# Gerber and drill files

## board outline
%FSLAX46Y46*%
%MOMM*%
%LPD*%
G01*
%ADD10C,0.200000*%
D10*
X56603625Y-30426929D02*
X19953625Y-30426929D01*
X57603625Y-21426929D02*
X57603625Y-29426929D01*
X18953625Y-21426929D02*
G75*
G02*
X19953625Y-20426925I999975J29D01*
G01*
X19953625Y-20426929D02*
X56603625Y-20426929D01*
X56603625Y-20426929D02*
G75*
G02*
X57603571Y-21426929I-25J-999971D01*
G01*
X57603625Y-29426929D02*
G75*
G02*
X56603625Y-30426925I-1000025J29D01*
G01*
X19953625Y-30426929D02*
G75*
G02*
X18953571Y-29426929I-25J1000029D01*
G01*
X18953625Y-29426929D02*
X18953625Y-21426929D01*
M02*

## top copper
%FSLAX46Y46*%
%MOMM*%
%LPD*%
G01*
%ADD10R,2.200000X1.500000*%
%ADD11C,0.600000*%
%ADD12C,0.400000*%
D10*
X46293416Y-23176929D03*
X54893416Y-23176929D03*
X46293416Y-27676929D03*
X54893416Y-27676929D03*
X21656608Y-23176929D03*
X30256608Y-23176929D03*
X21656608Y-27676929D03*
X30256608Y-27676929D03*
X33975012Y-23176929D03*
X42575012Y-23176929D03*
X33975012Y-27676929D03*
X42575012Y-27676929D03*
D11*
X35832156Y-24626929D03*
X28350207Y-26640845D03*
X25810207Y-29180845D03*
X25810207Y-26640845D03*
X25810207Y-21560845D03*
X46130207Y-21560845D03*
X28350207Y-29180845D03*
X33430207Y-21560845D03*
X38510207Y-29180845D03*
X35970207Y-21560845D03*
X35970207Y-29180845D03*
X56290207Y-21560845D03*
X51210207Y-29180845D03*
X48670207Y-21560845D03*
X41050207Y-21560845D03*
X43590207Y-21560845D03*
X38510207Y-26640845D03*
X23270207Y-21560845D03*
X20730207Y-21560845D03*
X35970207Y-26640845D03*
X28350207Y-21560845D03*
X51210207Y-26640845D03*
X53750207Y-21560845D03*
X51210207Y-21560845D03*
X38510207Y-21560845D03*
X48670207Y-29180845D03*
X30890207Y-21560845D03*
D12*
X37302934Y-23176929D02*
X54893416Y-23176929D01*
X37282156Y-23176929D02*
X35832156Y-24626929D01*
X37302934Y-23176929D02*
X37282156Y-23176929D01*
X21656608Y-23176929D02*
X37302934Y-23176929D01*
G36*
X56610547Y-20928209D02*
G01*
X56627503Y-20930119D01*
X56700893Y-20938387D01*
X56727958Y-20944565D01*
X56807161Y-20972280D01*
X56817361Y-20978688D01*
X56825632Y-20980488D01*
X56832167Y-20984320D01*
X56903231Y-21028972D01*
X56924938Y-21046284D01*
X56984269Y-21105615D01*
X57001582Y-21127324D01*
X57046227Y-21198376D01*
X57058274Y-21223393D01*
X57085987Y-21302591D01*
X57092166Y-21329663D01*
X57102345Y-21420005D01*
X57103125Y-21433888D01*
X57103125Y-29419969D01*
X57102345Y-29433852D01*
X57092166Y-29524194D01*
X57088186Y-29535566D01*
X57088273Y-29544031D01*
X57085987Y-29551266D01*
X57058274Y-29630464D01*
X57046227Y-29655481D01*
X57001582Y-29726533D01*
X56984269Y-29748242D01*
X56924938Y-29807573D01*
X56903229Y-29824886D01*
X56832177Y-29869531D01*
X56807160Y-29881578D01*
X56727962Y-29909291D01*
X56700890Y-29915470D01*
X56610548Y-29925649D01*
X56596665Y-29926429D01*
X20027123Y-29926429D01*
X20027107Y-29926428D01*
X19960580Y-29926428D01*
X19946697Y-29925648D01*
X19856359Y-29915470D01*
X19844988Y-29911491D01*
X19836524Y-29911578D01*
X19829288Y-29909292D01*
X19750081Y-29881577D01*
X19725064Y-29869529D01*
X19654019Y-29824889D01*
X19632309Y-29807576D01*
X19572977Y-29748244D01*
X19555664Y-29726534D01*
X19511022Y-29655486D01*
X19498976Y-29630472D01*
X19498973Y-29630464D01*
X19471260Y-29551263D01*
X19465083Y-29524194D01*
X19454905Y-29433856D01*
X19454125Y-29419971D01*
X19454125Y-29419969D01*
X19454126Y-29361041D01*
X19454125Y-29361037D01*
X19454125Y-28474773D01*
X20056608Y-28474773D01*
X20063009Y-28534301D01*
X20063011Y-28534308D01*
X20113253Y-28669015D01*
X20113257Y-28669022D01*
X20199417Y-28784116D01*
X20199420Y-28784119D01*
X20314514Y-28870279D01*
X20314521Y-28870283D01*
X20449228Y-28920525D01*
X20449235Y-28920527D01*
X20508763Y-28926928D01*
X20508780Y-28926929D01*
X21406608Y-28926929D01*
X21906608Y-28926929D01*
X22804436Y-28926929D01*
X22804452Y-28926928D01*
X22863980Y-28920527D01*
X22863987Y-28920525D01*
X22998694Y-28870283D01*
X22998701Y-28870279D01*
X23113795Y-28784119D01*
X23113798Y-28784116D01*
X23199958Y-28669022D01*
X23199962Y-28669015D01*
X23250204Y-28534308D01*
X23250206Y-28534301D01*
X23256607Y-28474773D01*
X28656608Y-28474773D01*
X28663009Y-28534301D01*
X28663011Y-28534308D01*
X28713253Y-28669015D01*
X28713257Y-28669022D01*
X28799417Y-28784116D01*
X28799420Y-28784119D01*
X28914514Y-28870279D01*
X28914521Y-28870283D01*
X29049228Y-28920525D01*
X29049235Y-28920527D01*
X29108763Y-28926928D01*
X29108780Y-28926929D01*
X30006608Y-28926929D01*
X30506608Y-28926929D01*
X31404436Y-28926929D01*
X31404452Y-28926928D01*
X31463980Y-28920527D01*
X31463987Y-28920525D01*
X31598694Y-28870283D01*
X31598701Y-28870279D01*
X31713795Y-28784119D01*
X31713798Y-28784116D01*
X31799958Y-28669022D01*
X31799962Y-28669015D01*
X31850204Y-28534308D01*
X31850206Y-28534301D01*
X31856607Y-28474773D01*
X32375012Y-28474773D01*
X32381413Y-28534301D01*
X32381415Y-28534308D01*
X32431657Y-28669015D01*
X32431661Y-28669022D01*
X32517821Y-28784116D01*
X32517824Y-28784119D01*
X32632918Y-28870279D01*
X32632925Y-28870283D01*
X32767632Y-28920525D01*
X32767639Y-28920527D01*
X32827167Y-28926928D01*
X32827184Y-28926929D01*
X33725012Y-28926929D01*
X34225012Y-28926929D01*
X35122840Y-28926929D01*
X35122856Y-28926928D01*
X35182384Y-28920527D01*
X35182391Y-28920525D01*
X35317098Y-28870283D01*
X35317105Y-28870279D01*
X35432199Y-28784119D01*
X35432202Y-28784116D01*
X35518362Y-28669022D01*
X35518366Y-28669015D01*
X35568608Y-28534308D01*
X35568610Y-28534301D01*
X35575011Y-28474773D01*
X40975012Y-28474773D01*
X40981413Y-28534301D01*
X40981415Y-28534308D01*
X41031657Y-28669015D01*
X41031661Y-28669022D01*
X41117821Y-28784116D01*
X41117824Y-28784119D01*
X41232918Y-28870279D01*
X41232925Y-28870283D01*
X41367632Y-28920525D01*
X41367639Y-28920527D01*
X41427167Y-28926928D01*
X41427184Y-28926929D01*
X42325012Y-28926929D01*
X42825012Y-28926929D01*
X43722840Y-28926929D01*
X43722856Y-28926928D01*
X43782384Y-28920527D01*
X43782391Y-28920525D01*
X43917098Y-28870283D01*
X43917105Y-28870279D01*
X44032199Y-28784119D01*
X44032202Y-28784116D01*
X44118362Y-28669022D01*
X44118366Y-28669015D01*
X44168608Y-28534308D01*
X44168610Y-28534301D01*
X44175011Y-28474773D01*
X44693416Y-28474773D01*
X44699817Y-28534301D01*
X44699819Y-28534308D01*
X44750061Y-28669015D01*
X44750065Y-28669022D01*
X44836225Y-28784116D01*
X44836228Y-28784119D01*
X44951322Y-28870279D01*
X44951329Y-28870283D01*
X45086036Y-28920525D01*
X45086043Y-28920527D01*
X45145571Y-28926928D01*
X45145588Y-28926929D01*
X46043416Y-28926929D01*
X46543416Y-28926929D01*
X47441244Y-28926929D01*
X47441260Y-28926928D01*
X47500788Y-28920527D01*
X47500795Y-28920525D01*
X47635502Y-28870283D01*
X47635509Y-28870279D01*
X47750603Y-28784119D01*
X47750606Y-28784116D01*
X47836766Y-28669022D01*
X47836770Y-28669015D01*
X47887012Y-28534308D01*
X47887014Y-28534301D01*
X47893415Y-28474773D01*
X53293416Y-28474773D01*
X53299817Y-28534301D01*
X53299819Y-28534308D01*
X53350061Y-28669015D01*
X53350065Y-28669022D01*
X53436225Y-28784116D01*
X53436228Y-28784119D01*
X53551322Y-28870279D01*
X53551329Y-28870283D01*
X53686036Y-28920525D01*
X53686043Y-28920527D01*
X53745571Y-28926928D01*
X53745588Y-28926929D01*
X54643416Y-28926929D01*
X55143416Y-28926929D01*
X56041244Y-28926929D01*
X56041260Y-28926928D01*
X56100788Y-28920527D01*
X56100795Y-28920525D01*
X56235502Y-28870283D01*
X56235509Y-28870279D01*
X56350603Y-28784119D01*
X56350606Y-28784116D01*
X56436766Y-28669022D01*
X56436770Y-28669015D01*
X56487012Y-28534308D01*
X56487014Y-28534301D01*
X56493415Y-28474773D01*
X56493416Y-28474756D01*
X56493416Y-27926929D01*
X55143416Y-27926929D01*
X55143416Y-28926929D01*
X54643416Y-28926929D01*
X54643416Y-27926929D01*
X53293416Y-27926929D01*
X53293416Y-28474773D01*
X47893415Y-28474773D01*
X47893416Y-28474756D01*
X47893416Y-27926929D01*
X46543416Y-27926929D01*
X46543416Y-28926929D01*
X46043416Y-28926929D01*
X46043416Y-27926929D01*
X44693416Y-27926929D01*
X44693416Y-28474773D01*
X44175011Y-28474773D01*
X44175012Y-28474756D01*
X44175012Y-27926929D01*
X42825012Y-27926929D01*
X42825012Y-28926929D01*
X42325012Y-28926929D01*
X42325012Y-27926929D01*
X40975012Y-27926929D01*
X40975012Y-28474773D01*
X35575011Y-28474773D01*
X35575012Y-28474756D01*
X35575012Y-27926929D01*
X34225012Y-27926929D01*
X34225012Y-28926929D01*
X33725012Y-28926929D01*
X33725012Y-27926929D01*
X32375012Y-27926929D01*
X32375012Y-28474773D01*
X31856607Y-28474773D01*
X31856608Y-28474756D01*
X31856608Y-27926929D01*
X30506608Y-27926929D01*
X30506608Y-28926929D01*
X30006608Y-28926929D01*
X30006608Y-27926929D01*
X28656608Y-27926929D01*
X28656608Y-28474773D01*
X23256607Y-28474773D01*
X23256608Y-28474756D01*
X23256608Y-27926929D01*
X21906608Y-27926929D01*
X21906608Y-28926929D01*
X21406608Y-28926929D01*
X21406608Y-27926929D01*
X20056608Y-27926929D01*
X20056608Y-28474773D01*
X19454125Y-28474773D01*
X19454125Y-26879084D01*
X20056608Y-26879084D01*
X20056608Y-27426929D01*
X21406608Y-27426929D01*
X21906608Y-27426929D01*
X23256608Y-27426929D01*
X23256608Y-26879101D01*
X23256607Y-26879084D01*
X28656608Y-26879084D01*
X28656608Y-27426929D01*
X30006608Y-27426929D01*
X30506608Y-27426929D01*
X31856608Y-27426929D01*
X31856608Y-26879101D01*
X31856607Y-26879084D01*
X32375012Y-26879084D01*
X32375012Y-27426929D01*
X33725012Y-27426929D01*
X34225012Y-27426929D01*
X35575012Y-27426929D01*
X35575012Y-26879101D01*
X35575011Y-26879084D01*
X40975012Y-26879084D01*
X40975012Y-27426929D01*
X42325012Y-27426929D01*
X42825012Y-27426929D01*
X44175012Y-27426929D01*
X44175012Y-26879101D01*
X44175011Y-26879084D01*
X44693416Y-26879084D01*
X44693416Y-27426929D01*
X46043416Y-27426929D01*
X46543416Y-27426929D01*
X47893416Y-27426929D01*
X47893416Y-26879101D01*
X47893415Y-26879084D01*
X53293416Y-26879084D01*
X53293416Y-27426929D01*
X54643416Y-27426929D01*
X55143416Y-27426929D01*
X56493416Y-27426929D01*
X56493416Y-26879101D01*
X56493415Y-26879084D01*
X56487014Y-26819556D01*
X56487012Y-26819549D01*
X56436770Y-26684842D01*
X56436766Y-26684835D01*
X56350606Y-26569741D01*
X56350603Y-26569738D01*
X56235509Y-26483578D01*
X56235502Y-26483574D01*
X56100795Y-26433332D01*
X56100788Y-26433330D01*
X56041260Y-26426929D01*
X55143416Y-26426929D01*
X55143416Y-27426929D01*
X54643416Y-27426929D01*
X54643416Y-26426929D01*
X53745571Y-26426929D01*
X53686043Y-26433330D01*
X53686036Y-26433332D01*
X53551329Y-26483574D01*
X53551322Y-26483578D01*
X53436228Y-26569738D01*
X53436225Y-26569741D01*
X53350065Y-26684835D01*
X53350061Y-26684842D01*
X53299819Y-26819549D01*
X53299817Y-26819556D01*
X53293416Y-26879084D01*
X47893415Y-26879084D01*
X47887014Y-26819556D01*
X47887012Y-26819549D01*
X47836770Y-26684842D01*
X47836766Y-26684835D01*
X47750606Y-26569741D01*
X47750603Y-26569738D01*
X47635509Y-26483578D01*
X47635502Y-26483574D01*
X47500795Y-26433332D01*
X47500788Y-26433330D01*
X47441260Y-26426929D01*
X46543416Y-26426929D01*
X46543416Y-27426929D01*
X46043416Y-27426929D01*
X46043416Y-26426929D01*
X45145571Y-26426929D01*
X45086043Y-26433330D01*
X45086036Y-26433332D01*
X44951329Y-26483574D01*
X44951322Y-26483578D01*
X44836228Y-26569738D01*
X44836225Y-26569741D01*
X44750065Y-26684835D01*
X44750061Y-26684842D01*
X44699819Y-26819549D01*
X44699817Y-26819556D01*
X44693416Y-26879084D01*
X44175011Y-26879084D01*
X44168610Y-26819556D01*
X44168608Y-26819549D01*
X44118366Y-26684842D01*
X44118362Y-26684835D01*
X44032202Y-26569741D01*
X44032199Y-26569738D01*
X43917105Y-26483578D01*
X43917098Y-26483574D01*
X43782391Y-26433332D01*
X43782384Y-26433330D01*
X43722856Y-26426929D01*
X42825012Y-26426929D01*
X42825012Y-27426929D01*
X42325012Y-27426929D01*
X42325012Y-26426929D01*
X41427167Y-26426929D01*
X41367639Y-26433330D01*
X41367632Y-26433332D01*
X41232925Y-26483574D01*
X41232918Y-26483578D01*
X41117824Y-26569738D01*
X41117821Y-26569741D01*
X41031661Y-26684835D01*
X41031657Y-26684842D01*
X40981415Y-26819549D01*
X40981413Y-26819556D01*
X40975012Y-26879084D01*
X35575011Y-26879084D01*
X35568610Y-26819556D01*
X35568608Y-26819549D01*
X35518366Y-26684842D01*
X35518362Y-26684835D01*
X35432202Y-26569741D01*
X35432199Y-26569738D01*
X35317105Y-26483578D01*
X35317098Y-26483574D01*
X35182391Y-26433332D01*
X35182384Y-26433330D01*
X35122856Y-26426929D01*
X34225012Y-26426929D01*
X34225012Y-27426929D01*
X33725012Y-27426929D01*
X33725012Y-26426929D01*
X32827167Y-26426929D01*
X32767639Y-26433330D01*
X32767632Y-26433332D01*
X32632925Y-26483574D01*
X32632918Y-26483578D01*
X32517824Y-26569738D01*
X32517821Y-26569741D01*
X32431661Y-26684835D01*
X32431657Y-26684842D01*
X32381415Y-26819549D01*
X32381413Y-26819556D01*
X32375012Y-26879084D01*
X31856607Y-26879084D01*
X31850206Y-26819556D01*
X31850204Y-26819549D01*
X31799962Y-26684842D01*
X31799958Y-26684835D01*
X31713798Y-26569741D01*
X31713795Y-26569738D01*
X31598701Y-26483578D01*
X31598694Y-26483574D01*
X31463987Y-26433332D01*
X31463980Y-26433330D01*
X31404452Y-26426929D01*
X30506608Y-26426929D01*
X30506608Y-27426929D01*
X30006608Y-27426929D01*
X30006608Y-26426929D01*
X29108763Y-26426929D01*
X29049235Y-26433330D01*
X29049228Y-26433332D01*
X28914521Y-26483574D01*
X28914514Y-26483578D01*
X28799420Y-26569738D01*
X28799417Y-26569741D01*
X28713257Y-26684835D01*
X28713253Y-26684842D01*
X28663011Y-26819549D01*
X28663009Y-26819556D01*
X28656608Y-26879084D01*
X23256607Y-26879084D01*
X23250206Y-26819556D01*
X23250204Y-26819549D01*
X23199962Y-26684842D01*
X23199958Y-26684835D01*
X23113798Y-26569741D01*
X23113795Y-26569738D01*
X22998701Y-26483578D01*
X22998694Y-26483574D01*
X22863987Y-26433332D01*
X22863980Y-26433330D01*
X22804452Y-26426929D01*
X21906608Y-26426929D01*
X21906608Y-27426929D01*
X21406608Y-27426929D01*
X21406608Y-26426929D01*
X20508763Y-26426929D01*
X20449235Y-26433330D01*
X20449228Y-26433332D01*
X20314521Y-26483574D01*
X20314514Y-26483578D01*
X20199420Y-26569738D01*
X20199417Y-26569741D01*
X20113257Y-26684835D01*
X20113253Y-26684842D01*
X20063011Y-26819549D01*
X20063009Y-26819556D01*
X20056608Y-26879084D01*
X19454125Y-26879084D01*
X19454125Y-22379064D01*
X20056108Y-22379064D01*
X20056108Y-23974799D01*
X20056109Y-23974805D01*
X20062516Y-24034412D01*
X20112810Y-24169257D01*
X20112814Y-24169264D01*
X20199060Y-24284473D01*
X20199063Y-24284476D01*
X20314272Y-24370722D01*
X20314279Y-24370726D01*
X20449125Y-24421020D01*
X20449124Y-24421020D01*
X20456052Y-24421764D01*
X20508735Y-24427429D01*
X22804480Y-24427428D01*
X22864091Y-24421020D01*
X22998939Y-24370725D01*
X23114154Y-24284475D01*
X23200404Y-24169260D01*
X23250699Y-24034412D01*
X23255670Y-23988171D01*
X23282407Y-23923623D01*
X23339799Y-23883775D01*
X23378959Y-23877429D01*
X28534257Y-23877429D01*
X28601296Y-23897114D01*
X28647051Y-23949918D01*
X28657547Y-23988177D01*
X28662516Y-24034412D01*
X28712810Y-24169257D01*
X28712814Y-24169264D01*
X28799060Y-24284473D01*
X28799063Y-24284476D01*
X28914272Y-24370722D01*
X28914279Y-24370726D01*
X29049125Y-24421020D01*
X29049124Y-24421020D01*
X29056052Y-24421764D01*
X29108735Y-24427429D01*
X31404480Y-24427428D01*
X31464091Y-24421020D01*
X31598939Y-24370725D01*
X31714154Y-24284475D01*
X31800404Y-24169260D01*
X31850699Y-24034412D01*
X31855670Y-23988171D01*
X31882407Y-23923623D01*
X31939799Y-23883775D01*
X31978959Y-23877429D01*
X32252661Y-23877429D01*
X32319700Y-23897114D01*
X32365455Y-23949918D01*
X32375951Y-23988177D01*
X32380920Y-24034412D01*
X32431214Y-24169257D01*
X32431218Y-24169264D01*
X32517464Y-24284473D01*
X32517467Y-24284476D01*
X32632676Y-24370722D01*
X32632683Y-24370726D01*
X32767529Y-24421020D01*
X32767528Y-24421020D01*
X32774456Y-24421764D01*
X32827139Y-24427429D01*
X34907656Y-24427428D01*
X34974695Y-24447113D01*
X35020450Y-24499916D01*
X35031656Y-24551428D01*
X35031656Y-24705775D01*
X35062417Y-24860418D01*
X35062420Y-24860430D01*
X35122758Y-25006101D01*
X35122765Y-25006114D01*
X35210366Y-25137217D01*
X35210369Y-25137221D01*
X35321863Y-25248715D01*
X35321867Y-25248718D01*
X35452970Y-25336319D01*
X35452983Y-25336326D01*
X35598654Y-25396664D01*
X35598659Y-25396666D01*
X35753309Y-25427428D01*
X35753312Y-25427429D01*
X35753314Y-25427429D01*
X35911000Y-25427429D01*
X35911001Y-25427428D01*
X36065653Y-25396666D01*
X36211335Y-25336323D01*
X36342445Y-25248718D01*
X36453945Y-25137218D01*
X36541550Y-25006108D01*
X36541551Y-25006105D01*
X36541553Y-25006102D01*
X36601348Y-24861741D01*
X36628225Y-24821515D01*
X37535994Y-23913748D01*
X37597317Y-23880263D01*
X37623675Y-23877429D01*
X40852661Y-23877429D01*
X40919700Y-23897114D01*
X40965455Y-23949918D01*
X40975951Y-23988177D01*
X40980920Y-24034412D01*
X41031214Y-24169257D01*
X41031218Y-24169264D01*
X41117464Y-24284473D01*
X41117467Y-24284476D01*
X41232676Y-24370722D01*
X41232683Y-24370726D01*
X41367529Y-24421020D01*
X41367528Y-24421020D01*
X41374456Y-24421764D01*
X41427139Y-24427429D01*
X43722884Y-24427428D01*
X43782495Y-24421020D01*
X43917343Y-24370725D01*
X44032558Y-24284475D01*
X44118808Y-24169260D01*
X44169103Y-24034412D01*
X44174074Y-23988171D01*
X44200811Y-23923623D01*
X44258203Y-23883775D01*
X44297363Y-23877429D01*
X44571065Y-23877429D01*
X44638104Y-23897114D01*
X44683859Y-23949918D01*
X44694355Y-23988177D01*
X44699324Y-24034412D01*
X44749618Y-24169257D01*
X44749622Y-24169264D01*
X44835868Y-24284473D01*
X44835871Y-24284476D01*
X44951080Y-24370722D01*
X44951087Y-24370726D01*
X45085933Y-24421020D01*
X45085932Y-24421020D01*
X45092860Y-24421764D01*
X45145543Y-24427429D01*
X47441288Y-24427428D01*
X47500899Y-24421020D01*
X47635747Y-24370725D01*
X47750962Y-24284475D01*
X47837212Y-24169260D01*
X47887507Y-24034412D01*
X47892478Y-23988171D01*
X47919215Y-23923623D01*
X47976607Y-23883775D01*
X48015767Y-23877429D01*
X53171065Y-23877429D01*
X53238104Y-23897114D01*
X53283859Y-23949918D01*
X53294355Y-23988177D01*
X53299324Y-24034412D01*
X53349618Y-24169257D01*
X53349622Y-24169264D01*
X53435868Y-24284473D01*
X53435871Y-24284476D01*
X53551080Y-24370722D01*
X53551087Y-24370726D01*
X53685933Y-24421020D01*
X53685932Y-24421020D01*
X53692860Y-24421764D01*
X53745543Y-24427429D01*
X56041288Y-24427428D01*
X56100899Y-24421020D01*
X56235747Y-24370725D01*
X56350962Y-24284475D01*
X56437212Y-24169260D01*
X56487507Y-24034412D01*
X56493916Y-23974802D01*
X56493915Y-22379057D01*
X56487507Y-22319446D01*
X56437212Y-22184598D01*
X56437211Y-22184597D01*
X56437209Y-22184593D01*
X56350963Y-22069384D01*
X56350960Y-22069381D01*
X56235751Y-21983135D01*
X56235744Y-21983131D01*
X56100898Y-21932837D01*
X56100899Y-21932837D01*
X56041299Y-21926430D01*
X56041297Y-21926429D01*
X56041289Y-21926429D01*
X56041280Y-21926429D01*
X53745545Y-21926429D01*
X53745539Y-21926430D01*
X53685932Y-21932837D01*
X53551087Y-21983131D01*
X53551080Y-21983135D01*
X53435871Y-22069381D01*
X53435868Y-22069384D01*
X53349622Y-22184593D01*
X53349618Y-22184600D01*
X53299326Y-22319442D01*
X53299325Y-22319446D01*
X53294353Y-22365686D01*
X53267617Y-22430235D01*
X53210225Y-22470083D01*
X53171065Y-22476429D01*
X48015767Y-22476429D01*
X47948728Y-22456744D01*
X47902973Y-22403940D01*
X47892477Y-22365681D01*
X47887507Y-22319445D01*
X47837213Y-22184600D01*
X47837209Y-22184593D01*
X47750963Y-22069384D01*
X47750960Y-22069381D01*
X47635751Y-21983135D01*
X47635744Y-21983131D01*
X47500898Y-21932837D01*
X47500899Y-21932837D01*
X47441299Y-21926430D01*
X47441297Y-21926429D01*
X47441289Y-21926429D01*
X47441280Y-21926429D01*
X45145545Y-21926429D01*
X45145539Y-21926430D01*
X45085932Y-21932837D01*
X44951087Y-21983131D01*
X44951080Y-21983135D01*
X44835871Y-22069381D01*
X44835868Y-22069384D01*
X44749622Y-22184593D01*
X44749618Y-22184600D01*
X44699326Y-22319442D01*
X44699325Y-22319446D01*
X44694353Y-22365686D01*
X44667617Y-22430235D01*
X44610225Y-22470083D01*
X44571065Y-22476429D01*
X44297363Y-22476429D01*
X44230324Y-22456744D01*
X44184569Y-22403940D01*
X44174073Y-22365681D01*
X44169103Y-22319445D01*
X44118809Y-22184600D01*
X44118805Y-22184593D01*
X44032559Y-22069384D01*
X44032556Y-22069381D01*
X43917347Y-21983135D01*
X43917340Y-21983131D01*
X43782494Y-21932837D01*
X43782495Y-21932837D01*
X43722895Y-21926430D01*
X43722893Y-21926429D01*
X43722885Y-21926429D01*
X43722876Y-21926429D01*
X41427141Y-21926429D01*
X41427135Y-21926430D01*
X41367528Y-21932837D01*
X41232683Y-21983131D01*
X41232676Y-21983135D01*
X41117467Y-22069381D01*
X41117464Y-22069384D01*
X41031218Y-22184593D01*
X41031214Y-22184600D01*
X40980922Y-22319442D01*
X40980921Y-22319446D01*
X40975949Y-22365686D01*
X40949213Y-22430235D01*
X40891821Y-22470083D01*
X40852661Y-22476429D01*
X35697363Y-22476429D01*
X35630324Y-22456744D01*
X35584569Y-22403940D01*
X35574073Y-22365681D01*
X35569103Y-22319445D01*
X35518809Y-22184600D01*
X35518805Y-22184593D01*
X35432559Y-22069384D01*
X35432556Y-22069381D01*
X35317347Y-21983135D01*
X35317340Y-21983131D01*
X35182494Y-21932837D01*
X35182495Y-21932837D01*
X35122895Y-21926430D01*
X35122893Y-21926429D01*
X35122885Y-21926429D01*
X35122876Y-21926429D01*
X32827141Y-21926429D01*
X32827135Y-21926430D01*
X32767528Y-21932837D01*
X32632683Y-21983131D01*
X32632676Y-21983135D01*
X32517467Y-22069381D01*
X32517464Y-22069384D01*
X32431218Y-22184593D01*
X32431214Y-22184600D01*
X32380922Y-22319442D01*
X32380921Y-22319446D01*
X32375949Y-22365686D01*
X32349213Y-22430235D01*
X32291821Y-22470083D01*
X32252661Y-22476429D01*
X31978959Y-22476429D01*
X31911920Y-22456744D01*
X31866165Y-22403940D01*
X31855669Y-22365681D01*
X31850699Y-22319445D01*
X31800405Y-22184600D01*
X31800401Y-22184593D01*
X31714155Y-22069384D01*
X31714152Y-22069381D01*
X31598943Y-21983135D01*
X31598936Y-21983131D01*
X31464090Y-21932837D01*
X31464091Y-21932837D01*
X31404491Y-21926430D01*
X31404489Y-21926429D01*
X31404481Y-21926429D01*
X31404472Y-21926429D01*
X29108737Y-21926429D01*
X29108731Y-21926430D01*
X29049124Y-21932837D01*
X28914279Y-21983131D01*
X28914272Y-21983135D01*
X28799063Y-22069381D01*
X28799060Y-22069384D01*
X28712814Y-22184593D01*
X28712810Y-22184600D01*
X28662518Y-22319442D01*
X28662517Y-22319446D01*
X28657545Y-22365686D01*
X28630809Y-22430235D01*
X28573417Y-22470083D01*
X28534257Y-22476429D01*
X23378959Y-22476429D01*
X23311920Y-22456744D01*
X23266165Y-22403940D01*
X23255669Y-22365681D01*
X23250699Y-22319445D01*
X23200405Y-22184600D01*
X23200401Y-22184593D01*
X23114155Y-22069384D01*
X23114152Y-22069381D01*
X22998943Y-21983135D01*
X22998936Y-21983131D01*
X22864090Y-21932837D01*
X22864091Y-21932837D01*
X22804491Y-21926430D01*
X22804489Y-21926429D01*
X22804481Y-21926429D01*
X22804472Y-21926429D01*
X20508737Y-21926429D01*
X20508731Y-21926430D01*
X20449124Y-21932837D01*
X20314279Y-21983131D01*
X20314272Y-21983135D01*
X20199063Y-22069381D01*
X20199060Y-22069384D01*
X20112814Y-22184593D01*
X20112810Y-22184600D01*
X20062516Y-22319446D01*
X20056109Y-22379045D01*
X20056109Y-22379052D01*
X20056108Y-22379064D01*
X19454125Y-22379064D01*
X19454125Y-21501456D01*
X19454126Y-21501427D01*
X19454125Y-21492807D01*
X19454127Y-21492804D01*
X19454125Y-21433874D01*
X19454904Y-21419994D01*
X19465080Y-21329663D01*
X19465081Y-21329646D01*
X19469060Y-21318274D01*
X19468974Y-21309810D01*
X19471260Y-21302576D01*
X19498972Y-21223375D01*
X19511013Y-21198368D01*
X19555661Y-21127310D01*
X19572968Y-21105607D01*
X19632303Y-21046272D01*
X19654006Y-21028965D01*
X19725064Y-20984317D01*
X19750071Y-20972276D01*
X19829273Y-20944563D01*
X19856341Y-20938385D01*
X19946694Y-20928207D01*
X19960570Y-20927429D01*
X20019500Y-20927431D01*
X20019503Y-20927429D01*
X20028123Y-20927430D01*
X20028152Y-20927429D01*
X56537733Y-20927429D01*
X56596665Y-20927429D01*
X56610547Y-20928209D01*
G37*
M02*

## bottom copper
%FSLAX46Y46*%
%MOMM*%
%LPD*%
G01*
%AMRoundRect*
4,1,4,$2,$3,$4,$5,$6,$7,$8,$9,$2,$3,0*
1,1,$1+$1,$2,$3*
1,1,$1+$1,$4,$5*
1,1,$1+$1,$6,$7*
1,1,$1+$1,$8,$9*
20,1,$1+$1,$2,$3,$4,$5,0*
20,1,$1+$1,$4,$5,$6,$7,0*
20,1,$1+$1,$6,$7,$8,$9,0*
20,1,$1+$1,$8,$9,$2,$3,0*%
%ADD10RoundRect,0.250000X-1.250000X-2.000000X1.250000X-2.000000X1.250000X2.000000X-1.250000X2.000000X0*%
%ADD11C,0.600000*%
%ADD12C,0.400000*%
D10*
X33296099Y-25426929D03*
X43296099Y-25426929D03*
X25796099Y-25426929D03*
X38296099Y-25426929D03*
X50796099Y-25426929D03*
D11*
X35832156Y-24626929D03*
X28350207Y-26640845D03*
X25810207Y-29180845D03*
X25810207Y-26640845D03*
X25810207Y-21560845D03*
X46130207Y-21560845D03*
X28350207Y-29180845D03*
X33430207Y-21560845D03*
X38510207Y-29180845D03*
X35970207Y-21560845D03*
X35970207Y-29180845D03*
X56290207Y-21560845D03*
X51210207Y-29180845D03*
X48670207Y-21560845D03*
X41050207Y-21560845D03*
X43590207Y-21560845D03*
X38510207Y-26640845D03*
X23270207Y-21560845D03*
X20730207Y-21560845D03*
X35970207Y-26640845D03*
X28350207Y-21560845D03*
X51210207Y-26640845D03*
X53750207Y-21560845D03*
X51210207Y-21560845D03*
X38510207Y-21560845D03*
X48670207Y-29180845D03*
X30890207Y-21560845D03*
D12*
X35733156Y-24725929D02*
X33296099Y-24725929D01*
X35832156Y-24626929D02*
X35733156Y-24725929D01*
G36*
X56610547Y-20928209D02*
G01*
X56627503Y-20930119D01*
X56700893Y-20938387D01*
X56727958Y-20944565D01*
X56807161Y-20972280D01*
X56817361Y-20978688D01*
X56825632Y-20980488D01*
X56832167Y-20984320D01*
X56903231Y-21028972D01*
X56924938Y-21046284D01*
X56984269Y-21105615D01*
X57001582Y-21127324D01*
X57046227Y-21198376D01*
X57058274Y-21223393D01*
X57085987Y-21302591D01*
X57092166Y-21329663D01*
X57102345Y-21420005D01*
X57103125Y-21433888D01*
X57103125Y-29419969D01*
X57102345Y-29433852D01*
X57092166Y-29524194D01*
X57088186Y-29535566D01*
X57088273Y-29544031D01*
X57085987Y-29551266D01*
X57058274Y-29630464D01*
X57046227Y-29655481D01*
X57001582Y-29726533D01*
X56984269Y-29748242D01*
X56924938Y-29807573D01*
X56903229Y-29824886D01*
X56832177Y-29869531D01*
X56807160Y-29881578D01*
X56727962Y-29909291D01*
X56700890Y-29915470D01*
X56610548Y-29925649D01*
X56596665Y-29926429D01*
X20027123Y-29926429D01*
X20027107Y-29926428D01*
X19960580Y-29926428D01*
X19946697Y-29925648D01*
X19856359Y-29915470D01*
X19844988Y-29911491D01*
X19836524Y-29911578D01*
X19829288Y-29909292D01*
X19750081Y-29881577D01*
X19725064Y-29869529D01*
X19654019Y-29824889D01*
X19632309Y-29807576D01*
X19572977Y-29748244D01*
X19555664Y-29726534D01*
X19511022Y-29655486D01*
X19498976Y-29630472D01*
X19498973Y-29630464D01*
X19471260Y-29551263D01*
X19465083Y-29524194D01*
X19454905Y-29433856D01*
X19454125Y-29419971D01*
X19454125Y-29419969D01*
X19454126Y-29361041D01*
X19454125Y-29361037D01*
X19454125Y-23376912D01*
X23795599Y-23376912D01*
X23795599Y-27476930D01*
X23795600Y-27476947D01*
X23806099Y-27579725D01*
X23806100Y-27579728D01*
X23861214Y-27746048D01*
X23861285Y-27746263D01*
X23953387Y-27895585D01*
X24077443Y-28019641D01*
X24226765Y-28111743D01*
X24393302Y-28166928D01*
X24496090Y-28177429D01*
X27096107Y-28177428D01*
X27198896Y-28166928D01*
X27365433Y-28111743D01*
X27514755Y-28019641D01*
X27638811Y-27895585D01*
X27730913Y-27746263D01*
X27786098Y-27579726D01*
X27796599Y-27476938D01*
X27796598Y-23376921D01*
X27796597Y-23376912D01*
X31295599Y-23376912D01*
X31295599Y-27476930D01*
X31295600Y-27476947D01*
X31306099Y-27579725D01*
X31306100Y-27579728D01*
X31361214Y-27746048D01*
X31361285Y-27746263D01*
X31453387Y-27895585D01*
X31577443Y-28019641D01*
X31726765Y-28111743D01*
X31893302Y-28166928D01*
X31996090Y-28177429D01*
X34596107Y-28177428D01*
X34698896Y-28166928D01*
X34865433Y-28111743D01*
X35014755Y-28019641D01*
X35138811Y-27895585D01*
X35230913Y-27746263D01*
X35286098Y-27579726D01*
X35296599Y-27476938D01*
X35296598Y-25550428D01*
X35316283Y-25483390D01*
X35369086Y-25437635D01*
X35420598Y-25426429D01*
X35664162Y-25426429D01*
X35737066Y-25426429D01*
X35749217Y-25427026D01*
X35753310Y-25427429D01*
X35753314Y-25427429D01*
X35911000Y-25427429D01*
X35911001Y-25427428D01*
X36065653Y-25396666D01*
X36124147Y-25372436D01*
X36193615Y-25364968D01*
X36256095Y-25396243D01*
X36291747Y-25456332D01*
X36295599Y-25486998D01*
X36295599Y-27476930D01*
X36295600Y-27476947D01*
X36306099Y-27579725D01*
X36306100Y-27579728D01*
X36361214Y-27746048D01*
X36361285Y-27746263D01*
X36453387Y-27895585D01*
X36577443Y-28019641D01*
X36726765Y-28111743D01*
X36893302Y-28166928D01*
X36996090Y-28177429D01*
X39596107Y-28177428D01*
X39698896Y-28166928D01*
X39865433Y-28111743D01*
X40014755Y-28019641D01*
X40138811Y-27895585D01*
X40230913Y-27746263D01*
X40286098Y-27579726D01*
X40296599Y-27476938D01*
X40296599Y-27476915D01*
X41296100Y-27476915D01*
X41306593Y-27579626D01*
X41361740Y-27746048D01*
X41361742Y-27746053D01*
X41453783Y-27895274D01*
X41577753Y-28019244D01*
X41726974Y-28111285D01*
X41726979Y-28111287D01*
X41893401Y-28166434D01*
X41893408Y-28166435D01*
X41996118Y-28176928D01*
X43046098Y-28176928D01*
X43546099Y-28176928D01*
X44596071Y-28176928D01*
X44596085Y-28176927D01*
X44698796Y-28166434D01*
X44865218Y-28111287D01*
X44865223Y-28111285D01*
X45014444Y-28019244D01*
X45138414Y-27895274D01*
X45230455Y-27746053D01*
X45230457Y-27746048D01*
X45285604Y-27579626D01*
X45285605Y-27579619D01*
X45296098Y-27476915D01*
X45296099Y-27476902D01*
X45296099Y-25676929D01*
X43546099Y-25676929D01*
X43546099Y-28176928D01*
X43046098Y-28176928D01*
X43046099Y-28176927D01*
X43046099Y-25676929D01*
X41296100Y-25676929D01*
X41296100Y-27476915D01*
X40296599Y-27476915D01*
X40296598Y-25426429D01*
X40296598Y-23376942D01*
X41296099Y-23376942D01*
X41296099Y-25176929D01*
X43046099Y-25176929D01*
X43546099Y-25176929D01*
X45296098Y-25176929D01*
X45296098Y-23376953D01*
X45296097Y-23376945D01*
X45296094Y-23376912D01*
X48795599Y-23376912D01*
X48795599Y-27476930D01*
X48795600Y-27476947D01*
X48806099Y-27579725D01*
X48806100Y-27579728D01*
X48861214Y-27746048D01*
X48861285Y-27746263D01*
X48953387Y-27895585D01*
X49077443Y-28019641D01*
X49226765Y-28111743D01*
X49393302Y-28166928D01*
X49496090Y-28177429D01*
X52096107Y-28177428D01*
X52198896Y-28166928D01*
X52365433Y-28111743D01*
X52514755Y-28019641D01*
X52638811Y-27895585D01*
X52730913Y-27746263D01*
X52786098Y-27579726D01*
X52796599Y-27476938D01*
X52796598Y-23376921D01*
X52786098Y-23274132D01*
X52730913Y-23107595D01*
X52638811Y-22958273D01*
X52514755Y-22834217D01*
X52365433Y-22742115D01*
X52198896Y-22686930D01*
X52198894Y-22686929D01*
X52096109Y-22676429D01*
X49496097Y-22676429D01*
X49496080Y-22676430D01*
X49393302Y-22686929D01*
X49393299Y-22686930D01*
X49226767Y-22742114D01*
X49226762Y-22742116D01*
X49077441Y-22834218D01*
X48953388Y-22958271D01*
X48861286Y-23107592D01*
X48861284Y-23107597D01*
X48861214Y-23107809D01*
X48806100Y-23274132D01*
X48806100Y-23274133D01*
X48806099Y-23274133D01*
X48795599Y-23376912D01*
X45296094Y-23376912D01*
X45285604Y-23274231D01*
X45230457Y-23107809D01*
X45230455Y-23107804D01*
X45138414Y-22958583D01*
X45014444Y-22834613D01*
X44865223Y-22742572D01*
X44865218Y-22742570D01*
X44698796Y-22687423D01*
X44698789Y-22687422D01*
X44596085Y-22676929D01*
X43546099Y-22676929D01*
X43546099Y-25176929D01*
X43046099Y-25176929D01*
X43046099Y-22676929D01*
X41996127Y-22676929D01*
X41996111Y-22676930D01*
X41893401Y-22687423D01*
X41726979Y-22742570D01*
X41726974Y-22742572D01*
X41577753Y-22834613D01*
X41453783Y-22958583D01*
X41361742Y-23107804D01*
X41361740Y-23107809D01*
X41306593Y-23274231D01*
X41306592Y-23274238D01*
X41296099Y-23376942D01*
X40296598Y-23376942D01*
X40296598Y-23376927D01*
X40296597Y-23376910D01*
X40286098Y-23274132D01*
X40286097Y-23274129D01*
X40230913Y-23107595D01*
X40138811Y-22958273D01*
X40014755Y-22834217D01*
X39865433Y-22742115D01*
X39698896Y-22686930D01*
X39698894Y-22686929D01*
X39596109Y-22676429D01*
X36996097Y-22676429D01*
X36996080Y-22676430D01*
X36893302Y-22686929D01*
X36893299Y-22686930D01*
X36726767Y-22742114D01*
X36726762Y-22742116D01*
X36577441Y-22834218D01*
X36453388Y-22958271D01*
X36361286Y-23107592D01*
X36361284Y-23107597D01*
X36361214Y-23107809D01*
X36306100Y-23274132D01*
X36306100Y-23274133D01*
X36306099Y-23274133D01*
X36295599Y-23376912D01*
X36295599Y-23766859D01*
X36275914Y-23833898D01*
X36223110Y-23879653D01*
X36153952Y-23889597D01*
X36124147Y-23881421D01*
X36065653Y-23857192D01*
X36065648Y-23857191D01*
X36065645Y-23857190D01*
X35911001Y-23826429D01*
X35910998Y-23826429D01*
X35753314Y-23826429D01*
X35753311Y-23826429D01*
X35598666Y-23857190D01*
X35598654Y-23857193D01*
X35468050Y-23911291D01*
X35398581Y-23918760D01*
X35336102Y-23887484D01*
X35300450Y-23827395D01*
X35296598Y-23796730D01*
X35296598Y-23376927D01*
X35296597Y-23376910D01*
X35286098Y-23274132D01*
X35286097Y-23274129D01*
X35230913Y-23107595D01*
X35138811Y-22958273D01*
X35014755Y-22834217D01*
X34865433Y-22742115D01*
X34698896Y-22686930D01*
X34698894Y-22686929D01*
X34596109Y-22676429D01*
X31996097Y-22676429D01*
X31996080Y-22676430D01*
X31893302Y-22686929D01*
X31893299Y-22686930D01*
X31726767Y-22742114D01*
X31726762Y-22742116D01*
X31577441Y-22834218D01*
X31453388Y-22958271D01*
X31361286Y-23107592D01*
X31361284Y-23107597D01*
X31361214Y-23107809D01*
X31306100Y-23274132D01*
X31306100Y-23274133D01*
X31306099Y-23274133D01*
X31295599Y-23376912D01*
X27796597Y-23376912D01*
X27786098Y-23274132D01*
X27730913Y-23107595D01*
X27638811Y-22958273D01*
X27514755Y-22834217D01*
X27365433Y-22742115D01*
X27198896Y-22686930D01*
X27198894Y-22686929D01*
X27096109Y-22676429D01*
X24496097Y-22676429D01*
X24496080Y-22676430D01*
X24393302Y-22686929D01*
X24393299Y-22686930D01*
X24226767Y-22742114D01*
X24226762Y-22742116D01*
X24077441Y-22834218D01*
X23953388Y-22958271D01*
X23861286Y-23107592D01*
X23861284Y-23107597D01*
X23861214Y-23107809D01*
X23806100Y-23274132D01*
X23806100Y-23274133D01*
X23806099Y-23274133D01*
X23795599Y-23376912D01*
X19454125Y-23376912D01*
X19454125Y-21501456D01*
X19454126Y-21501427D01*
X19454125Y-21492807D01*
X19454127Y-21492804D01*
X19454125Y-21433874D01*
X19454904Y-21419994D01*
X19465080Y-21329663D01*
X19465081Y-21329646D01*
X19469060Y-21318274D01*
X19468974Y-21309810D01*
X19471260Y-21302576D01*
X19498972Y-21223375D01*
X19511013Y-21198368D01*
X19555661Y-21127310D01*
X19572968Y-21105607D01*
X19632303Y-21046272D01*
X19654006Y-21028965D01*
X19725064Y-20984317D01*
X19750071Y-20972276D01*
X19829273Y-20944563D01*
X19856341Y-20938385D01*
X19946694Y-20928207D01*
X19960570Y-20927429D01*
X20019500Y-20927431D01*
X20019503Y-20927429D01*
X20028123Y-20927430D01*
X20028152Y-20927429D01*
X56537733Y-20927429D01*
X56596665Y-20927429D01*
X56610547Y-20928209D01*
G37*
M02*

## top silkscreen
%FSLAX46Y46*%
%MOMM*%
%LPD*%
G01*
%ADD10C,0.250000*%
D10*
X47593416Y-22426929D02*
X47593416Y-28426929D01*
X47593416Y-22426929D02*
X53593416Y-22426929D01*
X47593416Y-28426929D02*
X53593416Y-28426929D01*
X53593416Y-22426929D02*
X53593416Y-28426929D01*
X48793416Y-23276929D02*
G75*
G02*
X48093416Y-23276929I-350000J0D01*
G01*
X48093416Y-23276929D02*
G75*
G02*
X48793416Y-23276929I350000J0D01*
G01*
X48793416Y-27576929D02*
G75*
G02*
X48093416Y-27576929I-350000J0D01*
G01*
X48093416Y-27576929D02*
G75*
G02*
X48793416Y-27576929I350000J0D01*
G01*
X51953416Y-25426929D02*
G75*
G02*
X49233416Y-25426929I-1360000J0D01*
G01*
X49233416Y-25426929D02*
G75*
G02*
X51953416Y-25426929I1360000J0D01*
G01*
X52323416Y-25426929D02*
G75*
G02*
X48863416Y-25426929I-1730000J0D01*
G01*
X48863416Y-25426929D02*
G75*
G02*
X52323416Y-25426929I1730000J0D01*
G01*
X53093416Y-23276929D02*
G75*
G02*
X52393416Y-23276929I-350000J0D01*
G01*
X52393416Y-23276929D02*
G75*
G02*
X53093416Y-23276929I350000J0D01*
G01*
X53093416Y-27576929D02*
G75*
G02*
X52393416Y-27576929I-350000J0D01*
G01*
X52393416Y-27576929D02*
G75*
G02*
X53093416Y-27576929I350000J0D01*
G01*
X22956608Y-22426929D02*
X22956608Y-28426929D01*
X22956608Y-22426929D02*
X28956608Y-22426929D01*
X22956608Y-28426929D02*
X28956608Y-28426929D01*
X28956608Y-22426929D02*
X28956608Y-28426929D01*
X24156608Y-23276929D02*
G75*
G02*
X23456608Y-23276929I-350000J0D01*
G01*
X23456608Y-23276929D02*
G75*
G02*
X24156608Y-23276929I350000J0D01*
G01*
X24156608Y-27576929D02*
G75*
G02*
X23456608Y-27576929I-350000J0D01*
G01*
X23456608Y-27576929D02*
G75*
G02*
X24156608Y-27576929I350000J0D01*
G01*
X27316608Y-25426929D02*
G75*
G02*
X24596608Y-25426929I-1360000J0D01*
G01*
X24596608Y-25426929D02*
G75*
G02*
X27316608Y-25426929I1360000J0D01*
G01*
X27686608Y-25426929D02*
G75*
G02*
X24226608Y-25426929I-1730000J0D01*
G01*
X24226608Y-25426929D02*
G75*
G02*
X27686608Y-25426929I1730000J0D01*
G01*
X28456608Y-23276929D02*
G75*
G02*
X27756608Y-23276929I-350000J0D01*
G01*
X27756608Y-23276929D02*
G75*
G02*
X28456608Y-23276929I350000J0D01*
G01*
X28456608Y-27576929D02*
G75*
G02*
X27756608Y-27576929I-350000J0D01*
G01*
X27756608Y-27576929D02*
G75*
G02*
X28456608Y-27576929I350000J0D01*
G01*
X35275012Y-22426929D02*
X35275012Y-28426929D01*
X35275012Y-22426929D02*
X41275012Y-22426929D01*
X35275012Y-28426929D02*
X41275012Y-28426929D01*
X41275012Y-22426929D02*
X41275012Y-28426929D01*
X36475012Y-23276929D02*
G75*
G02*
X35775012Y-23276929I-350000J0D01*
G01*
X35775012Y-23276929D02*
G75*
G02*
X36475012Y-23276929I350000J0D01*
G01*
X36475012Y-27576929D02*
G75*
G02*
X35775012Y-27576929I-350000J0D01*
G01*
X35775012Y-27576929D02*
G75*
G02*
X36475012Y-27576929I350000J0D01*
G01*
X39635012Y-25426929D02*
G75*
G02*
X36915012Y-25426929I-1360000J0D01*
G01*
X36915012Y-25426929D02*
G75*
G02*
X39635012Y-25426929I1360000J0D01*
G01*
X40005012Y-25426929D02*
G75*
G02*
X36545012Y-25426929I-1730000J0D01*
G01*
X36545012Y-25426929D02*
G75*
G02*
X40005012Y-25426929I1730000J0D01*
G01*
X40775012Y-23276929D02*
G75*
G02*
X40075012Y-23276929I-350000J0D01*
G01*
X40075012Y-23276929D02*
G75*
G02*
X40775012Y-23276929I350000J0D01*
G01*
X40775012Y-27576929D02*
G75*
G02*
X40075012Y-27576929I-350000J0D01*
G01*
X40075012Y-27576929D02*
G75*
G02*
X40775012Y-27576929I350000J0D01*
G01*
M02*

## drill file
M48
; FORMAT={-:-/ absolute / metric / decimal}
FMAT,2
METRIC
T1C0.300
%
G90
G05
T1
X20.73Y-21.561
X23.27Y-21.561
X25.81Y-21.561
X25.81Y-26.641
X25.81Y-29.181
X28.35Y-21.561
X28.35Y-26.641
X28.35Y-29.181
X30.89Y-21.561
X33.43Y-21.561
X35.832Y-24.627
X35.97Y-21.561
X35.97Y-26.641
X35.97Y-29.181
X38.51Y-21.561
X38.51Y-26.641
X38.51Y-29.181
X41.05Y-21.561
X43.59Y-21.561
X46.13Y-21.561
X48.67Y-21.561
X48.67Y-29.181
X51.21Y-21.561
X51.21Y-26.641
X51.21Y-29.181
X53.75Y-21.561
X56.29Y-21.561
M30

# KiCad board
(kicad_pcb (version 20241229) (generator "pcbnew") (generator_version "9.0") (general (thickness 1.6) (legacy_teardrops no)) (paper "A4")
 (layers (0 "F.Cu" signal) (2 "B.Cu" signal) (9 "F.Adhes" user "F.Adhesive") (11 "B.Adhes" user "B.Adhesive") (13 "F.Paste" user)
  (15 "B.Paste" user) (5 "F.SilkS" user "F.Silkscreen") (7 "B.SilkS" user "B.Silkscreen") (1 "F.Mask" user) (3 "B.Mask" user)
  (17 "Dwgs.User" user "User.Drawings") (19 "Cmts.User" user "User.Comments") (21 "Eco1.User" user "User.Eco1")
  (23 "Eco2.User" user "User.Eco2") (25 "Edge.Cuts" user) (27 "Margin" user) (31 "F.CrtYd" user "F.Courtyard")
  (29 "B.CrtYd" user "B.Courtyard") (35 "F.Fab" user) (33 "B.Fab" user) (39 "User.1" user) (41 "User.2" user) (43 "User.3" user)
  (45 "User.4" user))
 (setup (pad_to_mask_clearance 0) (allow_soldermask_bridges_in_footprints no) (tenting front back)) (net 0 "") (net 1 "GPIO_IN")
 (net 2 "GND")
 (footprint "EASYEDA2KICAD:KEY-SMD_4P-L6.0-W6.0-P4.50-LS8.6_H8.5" (layer "F.Cu") (at 50.593416 25.426929)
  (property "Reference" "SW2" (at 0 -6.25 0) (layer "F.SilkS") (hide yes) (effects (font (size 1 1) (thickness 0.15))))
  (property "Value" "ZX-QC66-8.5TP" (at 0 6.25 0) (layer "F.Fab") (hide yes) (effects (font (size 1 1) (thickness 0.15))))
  (fp_line (start -3 -3) (end -3 3) (stroke (width 0.25) (type solid)) (layer "F.SilkS"))
  (fp_line (start -3 -3) (end 3 -3) (stroke (width 0.25) (type solid)) (layer "F.SilkS"))
  (fp_line (start -3 3) (end 3 3) (stroke (width 0.25) (type solid)) (layer "F.SilkS"))
  (fp_line (start 3 -3) (end 3 3) (stroke (width 0.25) (type solid)) (layer "F.SilkS"))
  (fp_circle (center -2.15 -2.15) (end -1.8 -2.15) (stroke (width 0.25) (type solid)) (fill no) (layer "F.SilkS"))
  (fp_circle (center -2.15 2.15) (end -1.8 2.15) (stroke (width 0.25) (type solid)) (fill no) (layer "F.SilkS"))
  (fp_circle (center 0 0) (end 1.36 0) (stroke (width 0.25) (type solid)) (fill no) (layer "F.SilkS"))
  (fp_circle (center 0 0) (end 1.73 0) (stroke (width 0.25) (type solid)) (fill no) (layer "F.SilkS"))
  (fp_circle (center 2.15 -2.15) (end 2.5 -2.15) (stroke (width 0.25) (type solid)) (fill no) (layer "F.SilkS"))
  (fp_circle (center 2.15 2.15) (end 2.5 2.15) (stroke (width 0.25) (type solid)) (fill no) (layer "F.SilkS"))
  (pad "1" smd rect (at -4.3 -2.25) (size 2.2 1.5) (layers "F.Cu" "F.Mask" "F.Paste") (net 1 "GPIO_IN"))
  (pad "2" smd rect (at 4.3 -2.25) (size 2.2 1.5) (layers "F.Cu" "F.Mask" "F.Paste") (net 1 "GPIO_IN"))
  (pad "3" smd rect (at -4.3 2.25) (size 2.2 1.5) (layers "F.Cu" "F.Mask" "F.Paste") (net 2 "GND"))
  (pad "4" smd rect (at 4.3 2.25) (size 2.2 1.5) (layers "F.Cu" "F.Mask" "F.Paste") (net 2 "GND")))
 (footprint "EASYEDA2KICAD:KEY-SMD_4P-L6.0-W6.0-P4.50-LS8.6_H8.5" (layer "F.Cu") (at 25.956608 25.426929)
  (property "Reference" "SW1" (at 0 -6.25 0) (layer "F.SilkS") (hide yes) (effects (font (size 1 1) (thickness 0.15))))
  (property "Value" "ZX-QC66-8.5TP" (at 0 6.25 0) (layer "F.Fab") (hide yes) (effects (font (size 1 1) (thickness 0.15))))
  (fp_line (start -3 -3) (end -3 3) (stroke (width 0.25) (type solid)) (layer "F.SilkS"))
  (fp_line (start -3 -3) (end 3 -3) (stroke (width 0.25) (type solid)) (layer "F.SilkS"))
  (fp_line (start -3 3) (end 3 3) (stroke (width 0.25) (type solid)) (layer "F.SilkS"))
  (fp_line (start 3 -3) (end 3 3) (stroke (width 0.25) (type solid)) (layer "F.SilkS"))
  (fp_circle (center -2.15 -2.15) (end -1.8 -2.15) (stroke (width 0.25) (type solid)) (fill no) (layer "F.SilkS"))
  (fp_circle (center -2.15 2.15) (end -1.8 2.15) (stroke (width 0.25) (type solid)) (fill no) (layer "F.SilkS"))
  (fp_circle (center 0 0) (end 1.36 0) (stroke (width 0.25) (type solid)) (fill no) (layer "F.SilkS"))
  (fp_circle (center 0 0) (end 1.73 0) (stroke (width 0.25) (type solid)) (fill no) (layer "F.SilkS"))
  (fp_circle (center 2.15 -2.15) (end 2.5 -2.15) (stroke (width 0.25) (type solid)) (fill no) (layer "F.SilkS"))
  (fp_circle (center 2.15 2.15) (end 2.5 2.15) (stroke (width 0.25) (type solid)) (fill no) (layer "F.SilkS"))
  (pad "1" smd rect (at -4.3 -2.25) (size 2.2 1.5) (layers "F.Cu" "F.Mask" "F.Paste") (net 1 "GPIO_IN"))
  (pad "2" smd rect (at 4.3 -2.25) (size 2.2 1.5) (layers "F.Cu" "F.Mask" "F.Paste") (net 1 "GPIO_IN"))
  (pad "3" smd rect (at -4.3 2.25) (size 2.2 1.5) (layers "F.Cu" "F.Mask" "F.Paste") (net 2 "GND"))
  (pad "4" smd rect (at 4.3 2.25) (size 2.2 1.5) (layers "F.Cu" "F.Mask" "F.Paste") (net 2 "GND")))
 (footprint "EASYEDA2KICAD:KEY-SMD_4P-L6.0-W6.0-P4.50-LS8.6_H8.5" (layer "F.Cu") (at 38.275012 25.426929)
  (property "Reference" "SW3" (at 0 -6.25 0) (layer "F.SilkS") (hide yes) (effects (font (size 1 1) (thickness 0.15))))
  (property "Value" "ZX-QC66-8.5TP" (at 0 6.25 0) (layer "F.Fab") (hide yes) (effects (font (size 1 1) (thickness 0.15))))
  (fp_line (start -3 -3) (end -3 3) (stroke (width 0.25) (type solid)) (layer "F.SilkS"))
  (fp_line (start -3 -3) (end 3 -3) (stroke (width 0.25) (type solid)) (layer "F.SilkS"))
  (fp_line (start -3 3) (end 3 3) (stroke (width 0.25) (type solid)) (layer "F.SilkS"))
  (fp_line (start 3 -3) (end 3 3) (stroke (width 0.25) (type solid)) (layer "F.SilkS"))
  (fp_circle (center -2.15 -2.15) (end -1.8 -2.15) (stroke (width 0.25) (type solid)) (fill no) (layer "F.SilkS"))
  (fp_circle (center -2.15 2.15) (end -1.8 2.15) (stroke (width 0.25) (type solid)) (fill no) (layer "F.SilkS"))
  (fp_circle (center 0 0) (end 1.36 0) (stroke (width 0.25) (type solid)) (fill no) (layer "F.SilkS"))
  (fp_circle (center 0 0) (end 1.73 0) (stroke (width 0.25) (type solid)) (fill no) (layer "F.SilkS"))
  (fp_circle (center 2.15 -2.15) (end 2.5 -2.15) (stroke (width 0.25) (type solid)) (fill no) (layer "F.SilkS"))
  (fp_circle (center 2.15 2.15) (end 2.5 2.15) (stroke (width 0.25) (type solid)) (fill no) (layer "F.SilkS"))
  (pad "1" smd rect (at -4.3 -2.25) (size 2.2 1.5) (layers "F.Cu" "F.Mask" "F.Paste") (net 1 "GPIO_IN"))
  (pad "2" smd rect (at 4.3 -2.25) (size 2.2 1.5) (layers "F.Cu" "F.Mask" "F.Paste") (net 1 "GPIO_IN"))
  (pad "3" smd rect (at -4.3 2.25) (size 2.2 1.5) (layers "F.Cu" "F.Mask" "F.Paste") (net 2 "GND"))
  (pad "4" smd rect (at 4.3 2.25) (size 2.2 1.5) (layers "F.Cu" "F.Mask" "F.Paste") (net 2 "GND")))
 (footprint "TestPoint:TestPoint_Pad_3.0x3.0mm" (layer "B.Cu") (at 38.296099 25.426929)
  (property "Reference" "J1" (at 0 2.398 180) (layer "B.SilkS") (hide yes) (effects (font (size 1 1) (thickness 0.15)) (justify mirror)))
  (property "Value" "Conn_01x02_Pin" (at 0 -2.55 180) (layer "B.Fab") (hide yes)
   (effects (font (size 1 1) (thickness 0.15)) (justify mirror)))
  (pad "1" smd roundrect (at -5 0) (size 3 4.5) (layers "B.Cu" "B.Mask") (roundrect_rratio 0.08333333333) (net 1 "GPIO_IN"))
  (pad "2" smd roundrect (at 5 0) (size 3 4.5) (layers "B.Cu" "B.Mask") (roundrect_rratio 0.08333333333) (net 2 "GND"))
  (pad "3" smd roundrect (at -12.5 0) (size 3 4.5) (layers "B.Cu" "B.Mask") (roundrect_rratio 0.08333333333))
  (pad "3" smd roundrect (at 0 0) (size 3 4.5) (layers "B.Cu" "B.Mask") (roundrect_rratio 0.08333333333))
  (pad "3" smd roundrect (at 12.5 0) (size 3 4.5) (layers "B.Cu" "B.Mask") (roundrect_rratio 0.08333333333)))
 (gr_line (start 56.603625 30.426929) (end 19.953625 30.426929) (stroke (width 0.2) (type default)) (layer "Edge.Cuts"))
 (gr_line (start 57.603625 21.426929) (end 57.603625 29.426929) (stroke (width 0.2) (type default)) (layer "Edge.Cuts"))
 (gr_arc (start 18.953625 21.426929) (mid 19.246509 20.719812) (end 19.953625 20.426929) (stroke (width 0.2) (type default))
  (layer "Edge.Cuts"))
 (gr_line (start 19.953625 20.426929) (end 56.603625 20.426929) (stroke (width 0.2) (type default)) (layer "Edge.Cuts"))
 (gr_arc (start 56.603625 20.426929) (mid 57.310732 20.719822) (end 57.603625 21.426929) (stroke (width 0.2) (type default))
  (layer "Edge.Cuts"))
 (gr_arc (start 57.603625 29.426929) (mid 57.310732 30.134036) (end 56.603625 30.426929) (stroke (width 0.2) (type default))
  (layer "Edge.Cuts"))
 (gr_arc (start 19.953625 30.426929) (mid 19.246515 30.134037) (end 18.953625 29.426929) (stroke (width 0.2) (type default))
  (layer "Edge.Cuts"))
 (gr_line (start 18.953625 29.426929) (end 18.953625 21.426929) (stroke (width 0.2) (type default)) (layer "Edge.Cuts"))
 (segment (start 37.302934 23.176929) (end 54.893416 23.176929) (width 0.4) (layer "F.Cu") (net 1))
 (segment (start 37.282156 23.176929) (end 35.832156 24.626929) (width 0.4) (layer "F.Cu") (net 1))
 (segment (start 37.302934 23.176929) (end 37.282156 23.176929) (width 0.4) (layer "F.Cu") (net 1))
 (segment (start 21.656608 23.176929) (end 37.302934 23.176929) (width 0.4) (layer "F.Cu") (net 1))
 (via (at 35.832156 24.626929) (size 0.6) (drill 0.3) (layers "F.Cu" "B.Cu") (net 1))
 (segment (start 35.733156 24.725929) (end 33.296099 24.725929) (width 0.4) (layer "B.Cu") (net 1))
 (segment (start 35.832156 24.626929) (end 35.733156 24.725929) (width 0.4) (layer "B.Cu") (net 1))
 (via (at 28.350207 26.640845) (size 0.6) (drill 0.3) (layers "F.Cu" "B.Cu") (free yes) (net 2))
 (via (at 25.810207 29.180845) (size 0.6) (drill 0.3) (layers "F.Cu" "B.Cu") (free yes) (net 2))
 (via (at 25.810207 26.640845) (size 0.6) (drill 0.3) (layers "F.Cu" "B.Cu") (free yes) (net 2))
 (via (at 25.810207 21.560845) (size 0.6) (drill 0.3) (layers "F.Cu" "B.Cu") (free yes) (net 2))
 (via (at 46.130207 21.560845) (size 0.6) (drill 0.3) (layers "F.Cu" "B.Cu") (free yes) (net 2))
 (via (at 28.350207 29.180845) (size 0.6) (drill 0.3) (layers "F.Cu" "B.Cu") (free yes) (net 2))
 (via (at 33.430207 21.560845) (size 0.6) (drill 0.3) (layers "F.Cu" "B.Cu") (free yes) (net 2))
 (via (at 38.510207 29.180845) (size 0.6) (drill 0.3) (layers "F.Cu" "B.Cu") (free yes) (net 2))
 (via (at 35.970207 21.560845) (size 0.6) (drill 0.3) (layers "F.Cu" "B.Cu") (free yes) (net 2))
 (via (at 35.970207 29.180845) (size 0.6) (drill 0.3) (layers "F.Cu" "B.Cu") (free yes) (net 2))
 (via (at 56.290207 21.560845) (size 0.6) (drill 0.3) (layers "F.Cu" "B.Cu") (free yes) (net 2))
 (via (at 51.210207 29.180845) (size 0.6) (drill 0.3) (layers "F.Cu" "B.Cu") (free yes) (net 2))
 (via (at 48.670207 21.560845) (size 0.6) (drill 0.3) (layers "F.Cu" "B.Cu") (free yes) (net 2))
 (via (at 41.050207 21.560845) (size 0.6) (drill 0.3) (layers "F.Cu" "B.Cu") (free yes) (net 2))
 (via (at 43.590207 21.560845) (size 0.6) (drill 0.3) (layers "F.Cu" "B.Cu") (free yes) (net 2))
 (via (at 38.510207 26.640845) (size 0.6) (drill 0.3) (layers "F.Cu" "B.Cu") (free yes) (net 2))
 (via (at 23.270207 21.560845) (size 0.6) (drill 0.3) (layers "F.Cu" "B.Cu") (free yes) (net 2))
 (via (at 20.730207 21.560845) (size 0.6) (drill 0.3) (layers "F.Cu" "B.Cu") (free yes) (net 2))
 (via (at 35.970207 26.640845) (size 0.6) (drill 0.3) (layers "F.Cu" "B.Cu") (free yes) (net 2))
 (via (at 28.350207 21.560845) (size 0.6) (drill 0.3) (layers "F.Cu" "B.Cu") (free yes) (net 2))
 (via (at 51.210207 26.640845) (size 0.6) (drill 0.3) (layers "F.Cu" "B.Cu") (free yes) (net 2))
 (via (at 53.750207 21.560845) (size 0.6) (drill 0.3) (layers "F.Cu" "B.Cu") (free yes) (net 2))
 (via (at 51.210207 21.560845) (size 0.6) (drill 0.3) (layers "F.Cu" "B.Cu") (free yes) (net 2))
 (via (at 38.510207 21.560845) (size 0.6) (drill 0.3) (layers "F.Cu" "B.Cu") (free yes) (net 2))
 (via (at 48.670207 29.180845) (size 0.6) (drill 0.3) (layers "F.Cu" "B.Cu") (free yes) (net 2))
 (via (at 30.890207 21.560845) (size 0.6) (drill 0.3) (layers "F.Cu" "B.Cu") (free yes) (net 2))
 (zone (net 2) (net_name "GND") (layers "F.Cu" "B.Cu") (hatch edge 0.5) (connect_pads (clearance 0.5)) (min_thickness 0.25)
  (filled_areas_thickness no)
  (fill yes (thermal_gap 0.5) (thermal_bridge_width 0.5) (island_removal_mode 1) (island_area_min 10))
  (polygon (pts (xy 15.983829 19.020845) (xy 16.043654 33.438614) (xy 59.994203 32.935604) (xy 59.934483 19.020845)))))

